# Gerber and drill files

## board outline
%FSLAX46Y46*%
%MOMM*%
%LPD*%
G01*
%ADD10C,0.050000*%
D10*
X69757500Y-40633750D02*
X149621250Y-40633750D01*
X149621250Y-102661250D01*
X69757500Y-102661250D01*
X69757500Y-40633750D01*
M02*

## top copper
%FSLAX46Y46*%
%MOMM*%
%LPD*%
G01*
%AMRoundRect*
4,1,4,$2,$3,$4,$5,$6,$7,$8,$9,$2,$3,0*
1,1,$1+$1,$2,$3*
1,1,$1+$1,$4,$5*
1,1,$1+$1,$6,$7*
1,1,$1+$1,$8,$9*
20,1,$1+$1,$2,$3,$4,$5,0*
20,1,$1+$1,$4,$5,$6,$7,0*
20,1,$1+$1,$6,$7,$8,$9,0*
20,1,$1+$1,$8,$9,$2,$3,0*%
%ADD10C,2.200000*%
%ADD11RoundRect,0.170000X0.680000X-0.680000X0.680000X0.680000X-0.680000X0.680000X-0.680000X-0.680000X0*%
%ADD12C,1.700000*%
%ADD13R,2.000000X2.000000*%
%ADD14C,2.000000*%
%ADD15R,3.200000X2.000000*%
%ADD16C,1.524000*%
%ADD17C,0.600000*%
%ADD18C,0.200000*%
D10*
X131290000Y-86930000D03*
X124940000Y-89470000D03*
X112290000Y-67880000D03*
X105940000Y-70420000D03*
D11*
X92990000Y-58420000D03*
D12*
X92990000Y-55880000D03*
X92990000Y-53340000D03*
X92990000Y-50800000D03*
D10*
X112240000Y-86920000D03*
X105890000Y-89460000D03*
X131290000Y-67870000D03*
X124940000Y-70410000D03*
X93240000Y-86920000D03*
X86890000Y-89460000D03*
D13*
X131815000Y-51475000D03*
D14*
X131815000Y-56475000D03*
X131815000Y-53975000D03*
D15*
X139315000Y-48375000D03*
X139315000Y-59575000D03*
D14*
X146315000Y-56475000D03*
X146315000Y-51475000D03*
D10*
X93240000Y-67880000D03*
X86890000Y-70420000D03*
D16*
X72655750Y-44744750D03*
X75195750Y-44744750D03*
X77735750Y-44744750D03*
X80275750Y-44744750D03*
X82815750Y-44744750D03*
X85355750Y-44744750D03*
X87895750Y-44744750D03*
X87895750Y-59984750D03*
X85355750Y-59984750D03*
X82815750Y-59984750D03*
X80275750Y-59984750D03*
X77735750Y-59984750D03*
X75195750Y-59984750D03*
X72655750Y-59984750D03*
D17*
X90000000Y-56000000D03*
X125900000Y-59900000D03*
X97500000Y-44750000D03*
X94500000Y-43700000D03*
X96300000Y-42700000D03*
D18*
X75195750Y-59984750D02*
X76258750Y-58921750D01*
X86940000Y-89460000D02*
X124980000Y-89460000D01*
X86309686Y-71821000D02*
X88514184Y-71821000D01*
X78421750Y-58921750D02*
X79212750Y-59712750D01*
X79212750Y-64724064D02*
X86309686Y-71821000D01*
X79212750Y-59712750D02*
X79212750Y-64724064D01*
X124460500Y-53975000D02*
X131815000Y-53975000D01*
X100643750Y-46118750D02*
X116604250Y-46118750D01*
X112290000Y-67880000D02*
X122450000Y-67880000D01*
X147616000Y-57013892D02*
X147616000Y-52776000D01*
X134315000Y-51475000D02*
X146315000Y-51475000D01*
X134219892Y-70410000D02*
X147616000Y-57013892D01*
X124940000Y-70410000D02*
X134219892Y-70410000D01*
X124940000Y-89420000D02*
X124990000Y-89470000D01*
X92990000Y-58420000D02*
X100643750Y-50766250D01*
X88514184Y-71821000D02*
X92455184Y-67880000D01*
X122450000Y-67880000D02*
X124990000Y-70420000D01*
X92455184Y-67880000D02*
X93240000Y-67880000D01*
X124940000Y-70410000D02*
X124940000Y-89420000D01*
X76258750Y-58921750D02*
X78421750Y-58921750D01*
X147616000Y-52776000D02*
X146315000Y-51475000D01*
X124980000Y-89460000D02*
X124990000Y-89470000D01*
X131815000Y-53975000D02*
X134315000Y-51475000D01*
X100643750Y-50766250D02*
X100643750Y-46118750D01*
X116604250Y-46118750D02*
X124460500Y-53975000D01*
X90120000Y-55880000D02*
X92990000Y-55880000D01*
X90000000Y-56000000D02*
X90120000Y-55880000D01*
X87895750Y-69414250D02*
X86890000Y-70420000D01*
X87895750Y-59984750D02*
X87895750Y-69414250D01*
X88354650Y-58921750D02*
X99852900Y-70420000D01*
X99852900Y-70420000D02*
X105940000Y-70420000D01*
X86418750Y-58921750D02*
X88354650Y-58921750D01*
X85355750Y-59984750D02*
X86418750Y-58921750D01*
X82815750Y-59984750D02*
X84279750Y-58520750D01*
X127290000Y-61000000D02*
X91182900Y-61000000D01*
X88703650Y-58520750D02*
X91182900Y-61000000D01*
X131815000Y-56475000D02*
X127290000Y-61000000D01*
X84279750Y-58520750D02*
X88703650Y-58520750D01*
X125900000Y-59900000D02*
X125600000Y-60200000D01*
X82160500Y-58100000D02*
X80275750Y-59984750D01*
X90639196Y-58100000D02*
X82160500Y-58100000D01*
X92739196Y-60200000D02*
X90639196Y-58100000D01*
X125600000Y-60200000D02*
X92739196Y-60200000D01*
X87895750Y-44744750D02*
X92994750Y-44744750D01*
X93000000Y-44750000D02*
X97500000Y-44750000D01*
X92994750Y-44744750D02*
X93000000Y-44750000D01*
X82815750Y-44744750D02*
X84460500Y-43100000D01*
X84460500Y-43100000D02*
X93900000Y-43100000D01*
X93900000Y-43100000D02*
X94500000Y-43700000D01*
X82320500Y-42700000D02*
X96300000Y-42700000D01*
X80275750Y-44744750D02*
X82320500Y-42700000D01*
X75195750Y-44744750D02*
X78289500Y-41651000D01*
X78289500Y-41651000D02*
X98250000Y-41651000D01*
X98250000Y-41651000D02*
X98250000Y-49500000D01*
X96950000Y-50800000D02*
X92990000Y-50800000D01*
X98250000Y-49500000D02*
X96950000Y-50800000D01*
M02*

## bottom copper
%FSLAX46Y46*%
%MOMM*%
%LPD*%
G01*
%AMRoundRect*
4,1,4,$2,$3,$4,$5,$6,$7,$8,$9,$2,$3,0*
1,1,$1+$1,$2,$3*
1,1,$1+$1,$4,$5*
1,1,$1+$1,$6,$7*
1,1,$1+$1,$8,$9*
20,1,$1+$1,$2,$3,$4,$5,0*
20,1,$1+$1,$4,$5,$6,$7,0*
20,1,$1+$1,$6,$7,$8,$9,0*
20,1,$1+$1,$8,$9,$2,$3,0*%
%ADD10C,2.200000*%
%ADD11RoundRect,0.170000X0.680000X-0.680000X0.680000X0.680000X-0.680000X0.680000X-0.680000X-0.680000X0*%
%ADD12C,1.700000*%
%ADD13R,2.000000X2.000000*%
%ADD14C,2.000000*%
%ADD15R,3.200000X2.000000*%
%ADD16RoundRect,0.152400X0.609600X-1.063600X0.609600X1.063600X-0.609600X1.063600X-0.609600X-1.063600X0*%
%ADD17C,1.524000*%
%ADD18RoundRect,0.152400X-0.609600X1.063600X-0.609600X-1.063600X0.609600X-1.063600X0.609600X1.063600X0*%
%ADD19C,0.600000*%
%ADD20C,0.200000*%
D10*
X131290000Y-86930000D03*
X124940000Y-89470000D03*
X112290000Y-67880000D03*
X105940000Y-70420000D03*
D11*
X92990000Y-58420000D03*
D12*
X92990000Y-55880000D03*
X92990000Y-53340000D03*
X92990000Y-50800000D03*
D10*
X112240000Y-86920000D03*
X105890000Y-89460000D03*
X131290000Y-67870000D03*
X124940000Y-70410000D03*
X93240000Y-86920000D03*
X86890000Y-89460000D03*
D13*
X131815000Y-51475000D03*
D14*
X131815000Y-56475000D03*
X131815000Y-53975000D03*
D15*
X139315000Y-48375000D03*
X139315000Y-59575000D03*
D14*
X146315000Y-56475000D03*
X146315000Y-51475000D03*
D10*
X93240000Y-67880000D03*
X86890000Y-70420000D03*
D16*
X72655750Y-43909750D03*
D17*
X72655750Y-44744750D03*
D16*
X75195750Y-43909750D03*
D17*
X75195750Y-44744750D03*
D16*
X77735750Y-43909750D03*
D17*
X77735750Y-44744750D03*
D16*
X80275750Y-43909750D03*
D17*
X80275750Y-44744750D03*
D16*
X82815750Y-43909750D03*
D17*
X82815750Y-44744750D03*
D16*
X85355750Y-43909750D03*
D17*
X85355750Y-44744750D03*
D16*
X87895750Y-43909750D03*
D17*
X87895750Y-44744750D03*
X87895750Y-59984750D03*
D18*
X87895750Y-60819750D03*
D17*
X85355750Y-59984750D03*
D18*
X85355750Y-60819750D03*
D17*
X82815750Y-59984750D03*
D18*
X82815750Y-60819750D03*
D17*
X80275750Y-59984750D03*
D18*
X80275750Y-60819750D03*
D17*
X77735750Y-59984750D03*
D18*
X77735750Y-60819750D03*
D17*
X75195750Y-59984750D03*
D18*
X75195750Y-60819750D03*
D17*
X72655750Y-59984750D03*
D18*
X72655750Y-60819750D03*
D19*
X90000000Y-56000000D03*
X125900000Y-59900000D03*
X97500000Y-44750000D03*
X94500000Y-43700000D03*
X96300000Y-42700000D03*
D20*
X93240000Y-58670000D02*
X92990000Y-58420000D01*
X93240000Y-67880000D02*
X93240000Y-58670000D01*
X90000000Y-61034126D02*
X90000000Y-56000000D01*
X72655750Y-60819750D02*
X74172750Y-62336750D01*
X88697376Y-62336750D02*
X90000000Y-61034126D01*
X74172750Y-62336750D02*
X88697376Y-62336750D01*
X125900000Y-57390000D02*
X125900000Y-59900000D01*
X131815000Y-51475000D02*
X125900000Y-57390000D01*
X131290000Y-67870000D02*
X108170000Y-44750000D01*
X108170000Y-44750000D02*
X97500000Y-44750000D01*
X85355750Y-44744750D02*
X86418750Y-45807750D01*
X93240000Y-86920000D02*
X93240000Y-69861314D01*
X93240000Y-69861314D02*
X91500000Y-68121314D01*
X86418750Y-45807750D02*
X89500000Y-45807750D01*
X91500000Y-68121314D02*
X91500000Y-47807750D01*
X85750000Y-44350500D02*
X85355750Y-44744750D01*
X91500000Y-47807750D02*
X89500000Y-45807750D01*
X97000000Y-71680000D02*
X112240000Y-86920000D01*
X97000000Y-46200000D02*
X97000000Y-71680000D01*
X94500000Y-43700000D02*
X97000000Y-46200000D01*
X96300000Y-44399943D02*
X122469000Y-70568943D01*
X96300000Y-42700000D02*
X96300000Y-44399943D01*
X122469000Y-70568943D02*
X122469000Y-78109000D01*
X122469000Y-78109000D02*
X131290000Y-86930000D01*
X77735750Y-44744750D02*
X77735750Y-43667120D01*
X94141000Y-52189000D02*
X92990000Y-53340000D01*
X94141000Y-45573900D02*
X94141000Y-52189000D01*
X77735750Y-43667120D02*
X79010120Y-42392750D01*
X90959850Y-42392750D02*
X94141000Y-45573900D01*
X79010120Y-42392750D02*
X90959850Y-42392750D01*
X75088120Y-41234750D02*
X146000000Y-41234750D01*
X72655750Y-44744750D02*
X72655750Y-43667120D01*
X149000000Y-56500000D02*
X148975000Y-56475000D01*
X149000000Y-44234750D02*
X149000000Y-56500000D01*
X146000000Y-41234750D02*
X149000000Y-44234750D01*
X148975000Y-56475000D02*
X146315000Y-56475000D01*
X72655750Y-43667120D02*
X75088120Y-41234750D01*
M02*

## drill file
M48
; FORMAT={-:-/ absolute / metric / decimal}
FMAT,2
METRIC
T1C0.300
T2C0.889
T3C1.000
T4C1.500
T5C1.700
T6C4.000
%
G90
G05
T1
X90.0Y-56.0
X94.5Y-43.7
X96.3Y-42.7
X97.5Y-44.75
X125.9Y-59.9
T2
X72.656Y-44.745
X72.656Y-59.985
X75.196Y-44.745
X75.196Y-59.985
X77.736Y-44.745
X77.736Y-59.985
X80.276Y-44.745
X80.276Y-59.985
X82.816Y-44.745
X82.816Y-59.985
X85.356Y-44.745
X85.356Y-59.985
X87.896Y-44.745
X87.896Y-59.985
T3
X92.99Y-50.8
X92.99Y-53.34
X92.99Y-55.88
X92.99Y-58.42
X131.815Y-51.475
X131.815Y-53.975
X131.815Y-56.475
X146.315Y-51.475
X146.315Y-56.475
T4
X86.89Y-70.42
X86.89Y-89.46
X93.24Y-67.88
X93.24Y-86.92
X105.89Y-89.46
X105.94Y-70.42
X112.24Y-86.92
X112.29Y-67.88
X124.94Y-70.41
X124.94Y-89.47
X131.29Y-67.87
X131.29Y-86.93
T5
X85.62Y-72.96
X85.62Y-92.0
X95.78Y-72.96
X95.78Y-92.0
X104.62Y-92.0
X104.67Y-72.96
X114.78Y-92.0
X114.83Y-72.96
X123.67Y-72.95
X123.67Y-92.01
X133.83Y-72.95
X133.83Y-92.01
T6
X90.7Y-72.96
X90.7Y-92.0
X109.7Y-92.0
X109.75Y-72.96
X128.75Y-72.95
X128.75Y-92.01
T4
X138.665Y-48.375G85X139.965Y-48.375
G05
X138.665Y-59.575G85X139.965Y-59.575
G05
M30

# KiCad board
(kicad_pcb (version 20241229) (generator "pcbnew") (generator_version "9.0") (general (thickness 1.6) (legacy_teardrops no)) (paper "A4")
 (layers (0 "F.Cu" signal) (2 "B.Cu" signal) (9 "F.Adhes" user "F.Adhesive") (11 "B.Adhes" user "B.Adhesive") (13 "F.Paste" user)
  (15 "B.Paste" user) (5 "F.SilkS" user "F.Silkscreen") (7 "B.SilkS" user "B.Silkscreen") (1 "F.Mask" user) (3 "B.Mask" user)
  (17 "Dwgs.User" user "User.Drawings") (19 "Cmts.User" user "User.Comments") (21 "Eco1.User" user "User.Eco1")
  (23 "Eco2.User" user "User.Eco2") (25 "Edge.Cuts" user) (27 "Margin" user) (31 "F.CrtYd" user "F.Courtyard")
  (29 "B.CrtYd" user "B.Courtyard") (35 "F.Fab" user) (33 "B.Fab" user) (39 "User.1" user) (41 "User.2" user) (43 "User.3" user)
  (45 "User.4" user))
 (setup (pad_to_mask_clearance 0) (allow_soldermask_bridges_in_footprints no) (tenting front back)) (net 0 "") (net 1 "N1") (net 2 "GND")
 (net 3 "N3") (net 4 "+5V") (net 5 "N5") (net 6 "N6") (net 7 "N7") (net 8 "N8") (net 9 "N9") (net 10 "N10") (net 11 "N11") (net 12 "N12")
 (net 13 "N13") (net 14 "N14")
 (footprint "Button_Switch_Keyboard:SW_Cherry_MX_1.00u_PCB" (layer "F.Cu") (at 131.29 86.93)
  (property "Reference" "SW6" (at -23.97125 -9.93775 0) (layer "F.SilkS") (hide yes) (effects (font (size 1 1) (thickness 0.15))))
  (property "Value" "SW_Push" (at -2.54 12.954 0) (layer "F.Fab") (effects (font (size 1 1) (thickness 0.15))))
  (pad "" np_thru_hole circle (at -7.62 5.08) (size 1.7 1.7) (drill 1.7) (layers "*.Cu" "*.Mask"))
  (pad "" np_thru_hole circle (at -2.54 5.08) (size 4 4) (drill 4) (layers "*.Cu" "*.Mask"))
  (pad "" np_thru_hole circle (at 2.54 5.08) (size 1.7 1.7) (drill 1.7) (layers "*.Cu" "*.Mask"))
  (pad "1" thru_hole circle (at 0 0) (size 2.2 2.2) (drill 1.5) (layers "*.Cu" "*.Mask") (remove_unused_layers no) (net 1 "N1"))
  (pad "2" thru_hole circle (at -6.35 2.54) (size 2.2 2.2) (drill 1.5) (layers "*.Cu" "*.Mask") (remove_unused_layers no) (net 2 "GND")))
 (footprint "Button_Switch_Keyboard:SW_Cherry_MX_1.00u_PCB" (layer "F.Cu") (at 112.29 67.88)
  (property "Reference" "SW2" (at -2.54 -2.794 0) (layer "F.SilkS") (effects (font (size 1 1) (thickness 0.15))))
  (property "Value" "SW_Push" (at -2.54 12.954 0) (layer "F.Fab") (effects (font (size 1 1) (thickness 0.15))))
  (pad "" np_thru_hole circle (at -7.62 5.08) (size 1.7 1.7) (drill 1.7) (layers "*.Cu" "*.Mask"))
  (pad "" np_thru_hole circle (at -2.54 5.08) (size 4 4) (drill 4) (layers "*.Cu" "*.Mask"))
  (pad "" np_thru_hole circle (at 2.54 5.08) (size 1.7 1.7) (drill 1.7) (layers "*.Cu" "*.Mask"))
  (pad "1" thru_hole circle (at 0 0) (size 2.2 2.2) (drill 1.5) (layers "*.Cu" "*.Mask") (remove_unused_layers no) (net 2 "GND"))
  (pad "2" thru_hole circle (at -6.35 2.54) (size 2.2 2.2) (drill 1.5) (layers "*.Cu" "*.Mask") (remove_unused_layers no) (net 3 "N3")))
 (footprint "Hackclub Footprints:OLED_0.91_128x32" (layer "F.Cu") (at 92.99 58.42 90)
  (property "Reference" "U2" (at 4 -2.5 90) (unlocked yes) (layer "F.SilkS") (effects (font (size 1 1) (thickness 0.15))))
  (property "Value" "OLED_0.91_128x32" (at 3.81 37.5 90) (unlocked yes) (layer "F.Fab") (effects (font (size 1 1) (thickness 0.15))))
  (pad "1" thru_hole roundrect (at 0 0 90) (size 1.7 1.7) (drill 1) (layers "*.Cu" "*.Mask") (remove_unused_layers no)
   (roundrect_rratio 0.1) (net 2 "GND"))
  (pad "2" thru_hole circle (at 2.54 0 90) (size 1.7 1.7) (drill 1) (layers "*.Cu" "*.Mask") (remove_unused_layers no) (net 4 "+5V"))
  (pad "3" thru_hole circle (at 5.08 0 90) (size 1.7 1.7) (drill 1) (layers "*.Cu" "*.Mask") (remove_unused_layers no) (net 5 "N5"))
  (pad "4" thru_hole circle (at 7.62 0 90) (size 1.7 1.7) (drill 1) (layers "*.Cu" "*.Mask") (remove_unused_layers no) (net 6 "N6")))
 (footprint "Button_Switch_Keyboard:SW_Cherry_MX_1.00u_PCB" (layer "F.Cu") (at 112.24 86.92)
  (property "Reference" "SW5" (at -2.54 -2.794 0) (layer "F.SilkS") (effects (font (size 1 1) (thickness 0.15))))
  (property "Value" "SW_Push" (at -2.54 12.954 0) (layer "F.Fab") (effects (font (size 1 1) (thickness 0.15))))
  (pad "" np_thru_hole circle (at -7.62 5.08) (size 1.7 1.7) (drill 1.7) (layers "*.Cu" "*.Mask"))
  (pad "" np_thru_hole circle (at -2.54 5.08) (size 4 4) (drill 4) (layers "*.Cu" "*.Mask"))
  (pad "" np_thru_hole circle (at 2.54 5.08) (size 1.7 1.7) (drill 1.7) (layers "*.Cu" "*.Mask"))
  (pad "1" thru_hole circle (at 0 0) (size 2.2 2.2) (drill 1.5) (layers "*.Cu" "*.Mask") (remove_unused_layers no) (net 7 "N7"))
  (pad "2" thru_hole circle (at -6.35 2.54) (size 2.2 2.2) (drill 1.5) (layers "*.Cu" "*.Mask") (remove_unused_layers no) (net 2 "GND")))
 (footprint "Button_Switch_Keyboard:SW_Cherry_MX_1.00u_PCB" (layer "F.Cu") (at 131.29 67.87)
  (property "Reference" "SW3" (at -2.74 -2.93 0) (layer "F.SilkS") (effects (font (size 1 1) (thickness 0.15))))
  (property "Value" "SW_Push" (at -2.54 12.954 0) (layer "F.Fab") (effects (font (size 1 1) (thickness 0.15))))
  (pad "" np_thru_hole circle (at -7.62 5.08) (size 1.7 1.7) (drill 1.7) (layers "*.Cu" "*.Mask"))
  (pad "" np_thru_hole circle (at -2.54 5.08) (size 4 4) (drill 4) (layers "*.Cu" "*.Mask"))
  (pad "" np_thru_hole circle (at 2.54 5.08) (size 1.7 1.7) (drill 1.7) (layers "*.Cu" "*.Mask"))
  (pad "1" thru_hole circle (at 0 0) (size 2.2 2.2) (drill 1.5) (layers "*.Cu" "*.Mask") (remove_unused_layers no) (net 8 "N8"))
  (pad "2" thru_hole circle (at -6.35 2.54) (size 2.2 2.2) (drill 1.5) (layers "*.Cu" "*.Mask") (remove_unused_layers no) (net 2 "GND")))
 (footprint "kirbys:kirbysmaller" (layer "F.Cu") (at 80 51.5)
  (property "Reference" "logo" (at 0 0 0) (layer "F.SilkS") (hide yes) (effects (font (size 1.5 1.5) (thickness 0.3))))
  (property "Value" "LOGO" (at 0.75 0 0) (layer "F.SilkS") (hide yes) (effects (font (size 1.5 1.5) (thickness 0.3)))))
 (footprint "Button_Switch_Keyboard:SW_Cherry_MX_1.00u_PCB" (layer "F.Cu") (at 93.24 86.92)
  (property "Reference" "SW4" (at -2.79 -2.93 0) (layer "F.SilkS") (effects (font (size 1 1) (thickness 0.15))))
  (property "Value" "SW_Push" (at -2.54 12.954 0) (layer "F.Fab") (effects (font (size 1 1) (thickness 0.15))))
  (pad "" np_thru_hole circle (at -7.62 5.08) (size 1.7 1.7) (drill 1.7) (layers "*.Cu" "*.Mask"))
  (pad "" np_thru_hole circle (at -2.54 5.08) (size 4 4) (drill 4) (layers "*.Cu" "*.Mask"))
  (pad "" np_thru_hole circle (at 2.54 5.08) (size 1.7 1.7) (drill 1.7) (layers "*.Cu" "*.Mask"))
  (pad "1" thru_hole circle (at 0 0) (size 2.2 2.2) (drill 1.5) (layers "*.Cu" "*.Mask") (remove_unused_layers no) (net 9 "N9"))
  (pad "2" thru_hole circle (at -6.35 2.54) (size 2.2 2.2) (drill 1.5) (layers "*.Cu" "*.Mask") (remove_unused_layers no) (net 2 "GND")))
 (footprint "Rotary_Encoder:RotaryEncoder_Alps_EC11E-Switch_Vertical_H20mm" (layer "F.Cu") (at 131.815 51.475)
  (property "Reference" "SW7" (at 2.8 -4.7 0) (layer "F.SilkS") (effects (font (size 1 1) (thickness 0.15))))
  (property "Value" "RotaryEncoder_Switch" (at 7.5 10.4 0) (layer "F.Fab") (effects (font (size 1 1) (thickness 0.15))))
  (pad "A" thru_hole rect (at 0 0) (size 2 2) (drill 1) (layers "*.Cu" "*.Mask") (remove_unused_layers no) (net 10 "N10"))
  (pad "B" thru_hole circle (at 0 5) (size 2 2) (drill 1) (layers "*.Cu" "*.Mask") (remove_unused_layers no) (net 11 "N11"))
  (pad "C" thru_hole circle (at 0 2.5) (size 2 2) (drill 1) (layers "*.Cu" "*.Mask") (remove_unused_layers no) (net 2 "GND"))
  (pad "MP" thru_hole rect (at 7.5 -3.1) (size 3.2 2) (drill oval 2.8 1.5) (layers "*.Cu" "*.Mask") (remove_unused_layers no))
  (pad "MP" thru_hole rect (at 7.5 8.1) (size 3.2 2) (drill oval 2.8 1.5) (layers "*.Cu" "*.Mask") (remove_unused_layers no))
  (pad "S1" thru_hole circle (at 14.5 5) (size 2 2) (drill 1) (layers "*.Cu" "*.Mask") (remove_unused_layers no) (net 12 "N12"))
  (pad "S2" thru_hole circle (at 14.5 0) (size 2 2) (drill 1) (layers "*.Cu" "*.Mask") (remove_unused_layers no) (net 2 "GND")))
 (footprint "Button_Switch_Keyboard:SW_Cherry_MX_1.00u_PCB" (layer "F.Cu") (at 93.24 67.88)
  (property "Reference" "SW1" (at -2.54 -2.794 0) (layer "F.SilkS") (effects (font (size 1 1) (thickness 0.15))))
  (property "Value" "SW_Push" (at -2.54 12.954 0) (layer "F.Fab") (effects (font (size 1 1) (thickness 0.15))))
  (pad "" np_thru_hole circle (at -7.62 5.08) (size 1.7 1.7) (drill 1.7) (layers "*.Cu" "*.Mask"))
  (pad "" np_thru_hole circle (at -2.54 5.08) (size 4 4) (drill 4) (layers "*.Cu" "*.Mask"))
  (pad "" np_thru_hole circle (at 2.54 5.08) (size 1.7 1.7) (drill 1.7) (layers "*.Cu" "*.Mask"))
  (pad "1" thru_hole circle (at 0 0) (size 2.2 2.2) (drill 1.5) (layers "*.Cu" "*.Mask") (remove_unused_layers no) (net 2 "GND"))
  (pad "2" thru_hole circle (at -6.35 2.54) (size 2.2 2.2) (drill 1.5) (layers "*.Cu" "*.Mask") (remove_unused_layers no) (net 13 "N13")))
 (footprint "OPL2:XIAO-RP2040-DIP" (layer "B.Cu") (at 80.27575 52.36475 -90)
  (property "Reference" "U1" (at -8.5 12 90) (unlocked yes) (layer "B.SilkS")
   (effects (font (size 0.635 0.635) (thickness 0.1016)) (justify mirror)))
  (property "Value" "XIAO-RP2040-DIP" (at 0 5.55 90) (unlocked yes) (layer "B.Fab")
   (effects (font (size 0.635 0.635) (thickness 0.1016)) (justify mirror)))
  (pad "1" smd roundrect (at -8.455 7.62 90) (size 2.432 1.524) (layers "B.Cu" "B.Mask") (roundrect_rratio 0.1) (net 12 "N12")
   (thermal_bridge_angle 45))
  (pad "1" thru_hole circle (at -7.62 7.62 90) (size 1.524 1.524) (drill 0.889) (layers "*.Cu" "*.Mask") (remove_unused_layers no)
   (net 12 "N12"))
  (pad "2" smd roundrect (at -8.455 5.08 90) (size 2.432 1.524) (layers "B.Cu" "B.Mask") (roundrect_rratio 0.1) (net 6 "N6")
   (thermal_bridge_angle 45))
  (pad "2" thru_hole circle (at -7.62 5.08 90) (size 1.524 1.524) (drill 0.889) (layers "*.Cu" "*.Mask") (remove_unused_layers no)
   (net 6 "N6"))
  (pad "3" smd roundrect (at -8.455 2.54 90) (size 2.432 1.524) (layers "B.Cu" "B.Mask") (roundrect_rratio 0.1) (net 5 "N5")
   (thermal_bridge_angle 45))
  (pad "3" thru_hole circle (at -7.62 2.54 90) (size 1.524 1.524) (drill 0.889) (layers "*.Cu" "*.Mask") (remove_unused_layers no)
   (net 5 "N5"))
  (pad "4" smd roundrect (at -8.455 0 90) (size 2.432 1.524) (layers "B.Cu" "B.Mask") (roundrect_rratio 0.1) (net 1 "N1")
   (thermal_bridge_angle 45))
  (pad "4" thru_hole circle (at -7.62 0 90) (size 1.524 1.524) (drill 0.889) (layers "*.Cu" "*.Mask") (remove_unused_layers no) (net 1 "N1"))
  (pad "5" smd roundrect (at -8.455 -2.54 90) (size 2.432 1.524) (layers "B.Cu" "B.Mask") (roundrect_rratio 0.1) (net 7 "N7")
   (thermal_bridge_angle 45))
  (pad "5" thru_hole circle (at -7.62 -2.54 90) (size 1.524 1.524) (drill 0.889) (layers "*.Cu" "*.Mask") (remove_unused_layers no)
   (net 7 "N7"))
  (pad "6" smd roundrect (at -8.455 -5.08 90) (size 2.432 1.524) (layers "B.Cu" "B.Mask") (roundrect_rratio 0.1) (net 9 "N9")
   (thermal_bridge_angle 45))
  (pad "6" thru_hole circle (at -7.62 -5.08 90) (size 1.524 1.524) (drill 0.889) (layers "*.Cu" "*.Mask") (remove_unused_layers no)
   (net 9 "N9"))
  (pad "7" smd roundrect (at -8.455 -7.62 90) (size 2.432 1.524) (layers "B.Cu" "B.Mask") (roundrect_rratio 0.1) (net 8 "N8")
   (thermal_bridge_angle 45))
  (pad "7" thru_hole circle (at -7.62 -7.62 90) (size 1.524 1.524) (drill 0.889) (layers "*.Cu" "*.Mask") (remove_unused_layers no)
   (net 8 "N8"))
  (pad "8" thru_hole circle (at 7.62 -7.62 270) (size 1.524 1.524) (drill 0.889) (layers "*.Cu" "*.Mask") (remove_unused_layers no)
   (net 13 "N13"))
  (pad "8" smd roundrect (at 8.455 -7.62 270) (size 2.432 1.524) (layers "B.Cu" "B.Mask") (roundrect_rratio 0.1) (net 13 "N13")
   (thermal_bridge_angle 45))
  (pad "9" thru_hole circle (at 7.62 -5.08 270) (size 1.524 1.524) (drill 0.889) (layers "*.Cu" "*.Mask") (remove_unused_layers no)
   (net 3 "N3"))
  (pad "9" smd roundrect (at 8.455 -5.08 270) (size 2.432 1.524) (layers "B.Cu" "B.Mask") (roundrect_rratio 0.1) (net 3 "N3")
   (thermal_bridge_angle 45))
  (pad "10" thru_hole circle (at 7.62 -2.54 270) (size 1.524 1.524) (drill 0.889) (layers "*.Cu" "*.Mask") (remove_unused_layers no)
   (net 11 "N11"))
  (pad "10" smd roundrect (at 8.455 -2.54 270) (size 2.432 1.524) (layers "B.Cu" "B.Mask") (roundrect_rratio 0.1) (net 11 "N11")
   (thermal_bridge_angle 45))
  (pad "11" thru_hole circle (at 7.62 0 270) (size 1.524 1.524) (drill 0.889) (layers "*.Cu" "*.Mask") (remove_unused_layers no)
   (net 10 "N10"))
  (pad "11" smd roundrect (at 8.455 0 270) (size 2.432 1.524) (layers "B.Cu" "B.Mask") (roundrect_rratio 0.1) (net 10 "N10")
   (thermal_bridge_angle 45))
  (pad "12" thru_hole circle (at 7.62 2.54 270) (size 1.524 1.524) (drill 0.889) (layers "*.Cu" "*.Mask") (remove_unused_layers no)
   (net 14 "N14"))
  (pad "12" smd roundrect (at 8.455 2.54 270) (size 2.432 1.524) (layers "B.Cu" "B.Mask") (roundrect_rratio 0.1) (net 14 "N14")
   (thermal_bridge_angle 45))
  (pad "13" thru_hole circle (at 7.62 5.08 270) (size 1.524 1.524) (drill 0.889) (layers "*.Cu" "*.Mask") (remove_unused_layers no)
   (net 2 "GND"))
  (pad "13" smd roundrect (at 8.455 5.08 270) (size 2.432 1.524) (layers "B.Cu" "B.Mask") (roundrect_rratio 0.1) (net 2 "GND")
   (thermal_bridge_angle 45))
  (pad "14" thru_hole circle (at 7.62 7.62 270) (size 1.524 1.524) (drill 0.889) (layers "*.Cu" "*.Mask") (remove_unused_layers no)
   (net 4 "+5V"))
  (pad "14" smd roundrect (at 8.455 7.62 270) (size 2.432 1.524) (layers "B.Cu" "B.Mask") (roundrect_rratio 0.1) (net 4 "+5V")
   (thermal_bridge_angle 45)))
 (gr_rect (start 69.7575 40.63375) (end 149.62125 102.66125) (stroke (width 0.05) (type default)) (fill no) (layer "Edge.Cuts"))
 (segment (start 75.19575 59.98475) (end 76.25875 58.92175) (width 0.2) (layer "F.Cu") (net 2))
 (segment (start 86.94 89.46) (end 124.98 89.46) (width 0.2) (layer "F.Cu") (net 2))
 (segment (start 86.309686 71.821) (end 88.514184 71.821) (width 0.2) (layer "F.Cu") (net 2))
 (segment (start 78.42175 58.92175) (end 79.21275 59.71275) (width 0.2) (layer "F.Cu") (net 2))
 (segment (start 79.21275 64.724064) (end 86.309686 71.821) (width 0.2) (layer "F.Cu") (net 2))
 (segment (start 79.21275 59.71275) (end 79.21275 64.724064) (width 0.2) (layer "F.Cu") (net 2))
 (segment (start 124.4605 53.975) (end 131.815 53.975) (width 0.2) (layer "F.Cu") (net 2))
 (segment (start 100.64375 46.11875) (end 116.60425 46.11875) (width 0.2) (layer "F.Cu") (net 2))
 (segment (start 112.29 67.88) (end 122.45 67.88) (width 0.2) (layer "F.Cu") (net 2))
 (segment (start 147.616 57.013892) (end 147.616 52.776) (width 0.2) (layer "F.Cu") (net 2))
 (segment (start 134.315 51.475) (end 146.315 51.475) (width 0.2) (layer "F.Cu") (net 2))
 (segment (start 134.219892 70.41) (end 147.616 57.013892) (width 0.2) (layer "F.Cu") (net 2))
 (segment (start 124.94 70.41) (end 134.219892 70.41) (width 0.2) (layer "F.Cu") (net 2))
 (segment (start 124.94 89.42) (end 124.99 89.47) (width 0.2) (layer "F.Cu") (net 2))
 (segment (start 92.99 58.42) (end 100.64375 50.76625) (width 0.2) (layer "F.Cu") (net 2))
 (segment (start 88.514184 71.821) (end 92.455184 67.88) (width 0.2) (layer "F.Cu") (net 2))
 (segment (start 122.45 67.88) (end 124.99 70.42) (width 0.2) (layer "F.Cu") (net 2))
 (segment (start 92.455184 67.88) (end 93.24 67.88) (width 0.2) (layer "F.Cu") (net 2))
 (segment (start 124.94 70.41) (end 124.94 89.42) (width 0.2) (layer "F.Cu") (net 2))
 (segment (start 76.25875 58.92175) (end 78.42175 58.92175) (width 0.2) (layer "F.Cu") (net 2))
 (segment (start 147.616 52.776) (end 146.315 51.475) (width 0.2) (layer "F.Cu") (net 2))
 (segment (start 124.98 89.46) (end 124.99 89.47) (width 0.2) (layer "F.Cu") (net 2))
 (segment (start 131.815 53.975) (end 134.315 51.475) (width 0.2) (layer "F.Cu") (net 2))
 (segment (start 100.64375 50.76625) (end 100.64375 46.11875) (width 0.2) (layer "F.Cu") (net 2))
 (segment (start 116.60425 46.11875) (end 124.4605 53.975) (width 0.2) (layer "F.Cu") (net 2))
 (segment (start 93.24 58.67) (end 92.99 58.42) (width 0.2) (layer "B.Cu") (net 2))
 (segment (start 93.24 67.88) (end 93.24 58.67) (width 0.2) (layer "B.Cu") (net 2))
 (segment (start 90.12 55.88) (end 92.99 55.88) (width 0.2) (layer "F.Cu") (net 4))
 (segment (start 90 56) (end 90.12 55.88) (width 0.2) (layer "F.Cu") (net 4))
 (via (at 90 56) (size 0.6) (drill 0.3) (layers "F.Cu" "B.Cu") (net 4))
 (segment (start 90 61.034126) (end 90 56) (width 0.2) (layer "B.Cu") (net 4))
 (segment (start 72.65575 60.81975) (end 74.17275 62.33675) (width 0.2) (layer "B.Cu") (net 4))
 (segment (start 88.697376 62.33675) (end 90 61.034126) (width 0.2) (layer "B.Cu") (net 4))
 (segment (start 74.17275 62.33675) (end 88.697376 62.33675) (width 0.2) (layer "B.Cu") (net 4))
 (segment (start 87.89575 69.41425) (end 86.89 70.42) (width 0.2) (layer "F.Cu") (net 13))
 (segment (start 87.89575 59.98475) (end 87.89575 69.41425) (width 0.2) (layer "F.Cu") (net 13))
 (segment (start 88.35465 58.92175) (end 99.8529 70.42) (width 0.2) (layer "F.Cu") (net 3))
 (segment (start 99.8529 70.42) (end 105.94 70.42) (width 0.2) (layer "F.Cu") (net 3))
 (segment (start 86.41875 58.92175) (end 88.35465 58.92175) (width 0.2) (layer "F.Cu") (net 3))
 (segment (start 85.35575 59.98475) (end 86.41875 58.92175) (width 0.2) (layer "F.Cu") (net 3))
 (segment (start 82.81575 59.98475) (end 84.27975 58.52075) (width 0.2) (layer "F.Cu") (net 11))
 (segment (start 127.29 61) (end 91.1829 61) (width 0.2) (layer "F.Cu") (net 11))
 (segment (start 88.70365 58.52075) (end 91.1829 61) (width 0.2) (layer "F.Cu") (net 11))
 (segment (start 131.815 56.475) (end 127.29 61) (width 0.2) (layer "F.Cu") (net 11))
 (segment (start 84.27975 58.52075) (end 88.70365 58.52075) (width 0.2) (layer "F.Cu") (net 11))
 (segment (start 125.9 59.9) (end 125.6 60.2) (width 0.2) (layer "F.Cu") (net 10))
 (segment (start 82.1605 58.1) (end 80.27575 59.98475) (width 0.2) (layer "F.Cu") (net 10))
 (segment (start 90.639196 58.1) (end 82.1605 58.1) (width 0.2) (layer "F.Cu") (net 10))
 (segment (start 92.739196 60.2) (end 90.639196 58.1) (width 0.2) (layer "F.Cu") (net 10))
 (segment (start 125.6 60.2) (end 92.739196 60.2) (width 0.2) (layer "F.Cu") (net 10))
 (via (at 125.9 59.9) (size 0.6) (drill 0.3) (layers "F.Cu" "B.Cu") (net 10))
 (segment (start 125.9 57.39) (end 125.9 59.9) (width 0.2) (layer "B.Cu") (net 10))
 (segment (start 131.815 51.475) (end 125.9 57.39) (width 0.2) (layer "B.Cu") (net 10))
 (segment (start 87.89575 44.74475) (end 92.99475 44.74475) (width 0.2) (layer "F.Cu") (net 8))
 (segment (start 93 44.75) (end 97.5 44.75) (width 0.2) (layer "F.Cu") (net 8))
 (segment (start 92.99475 44.74475) (end 93 44.75) (width 0.2) (layer "F.Cu") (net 8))
 (via (at 97.5 44.75) (size 0.6) (drill 0.3) (layers "F.Cu" "B.Cu") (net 8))
 (segment (start 131.29 67.87) (end 108.17 44.75) (width 0.2) (layer "B.Cu") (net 8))
 (segment (start 108.17 44.75) (end 97.5 44.75) (width 0.2) (layer "B.Cu") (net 8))
 (segment (start 85.35575 44.74475) (end 86.41875 45.80775) (width 0.2) (layer "B.Cu") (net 9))
 (segment (start 93.24 86.92) (end 93.24 69.861314) (width 0.2) (layer "B.Cu") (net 9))
 (segment (start 93.24 69.861314) (end 91.5 68.121314) (width 0.2) (layer "B.Cu") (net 9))
 (segment (start 86.41875 45.80775) (end 89.5 45.80775) (width 0.2) (layer "B.Cu") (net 9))
 (segment (start 91.5 68.121314) (end 91.5 47.80775) (width 0.2) (layer "B.Cu") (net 9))
 (segment (start 85.75 44.3505) (end 85.35575 44.74475) (width 0.2) (layer "B.Cu") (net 9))
 (segment (start 91.5 47.80775) (end 89.5 45.80775) (width 0.2) (layer "B.Cu") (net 9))
 (segment (start 82.81575 44.74475) (end 84.4605 43.1) (width 0.2) (layer "F.Cu") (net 7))
 (segment (start 84.4605 43.1) (end 93.9 43.1) (width 0.2) (layer "F.Cu") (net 7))
 (segment (start 93.9 43.1) (end 94.5 43.7) (width 0.2) (layer "F.Cu") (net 7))
 (via (at 94.5 43.7) (size 0.6) (drill 0.3) (layers "F.Cu" "B.Cu") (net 7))
 (segment (start 97 71.68) (end 112.24 86.92) (width 0.2) (layer "B.Cu") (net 7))
 (segment (start 97 46.2) (end 97 71.68) (width 0.2) (layer "B.Cu") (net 7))
 (segment (start 94.5 43.7) (end 97 46.2) (width 0.2) (layer "B.Cu") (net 7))
 (segment (start 82.3205 42.7) (end 96.3 42.7) (width 0.2) (layer "F.Cu") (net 1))
 (segment (start 80.27575 44.74475) (end 82.3205 42.7) (width 0.2) (layer "F.Cu") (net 1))
 (via (at 96.3 42.7) (size 0.6) (drill 0.3) (layers "F.Cu" "B.Cu") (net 1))
 (segment (start 96.3 44.399943) (end 122.469 70.568943) (width 0.2) (layer "B.Cu") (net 1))
 (segment (start 96.3 42.7) (end 96.3 44.399943) (width 0.2) (layer "B.Cu") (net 1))
 (segment (start 122.469 70.568943) (end 122.469 78.109) (width 0.2) (layer "B.Cu") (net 1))
 (segment (start 122.469 78.109) (end 131.29 86.93) (width 0.2) (layer "B.Cu") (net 1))
 (segment (start 77.73575 44.74475) (end 77.73575 43.66712) (width 0.2) (layer "B.Cu") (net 5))
 (segment (start 94.141 52.189) (end 92.99 53.34) (width 0.2) (layer "B.Cu") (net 5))
 (segment (start 94.141 45.5739) (end 94.141 52.189) (width 0.2) (layer "B.Cu") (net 5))
 (segment (start 77.73575 43.66712) (end 79.01012 42.39275) (width 0.2) (layer "B.Cu") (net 5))
 (segment (start 90.95985 42.39275) (end 94.141 45.5739) (width 0.2) (layer "B.Cu") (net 5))
 (segment (start 79.01012 42.39275) (end 90.95985 42.39275) (width 0.2) (layer "B.Cu") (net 5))
 (segment (start 75.19575 44.74475) (end 78.2895 41.651) (width 0.2) (layer "F.Cu") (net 6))
 (segment (start 78.2895 41.651) (end 98.25 41.651) (width 0.2) (layer "F.Cu") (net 6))
 (segment (start 98.25 41.651) (end 98.25 49.5) (width 0.2) (layer "F.Cu") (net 6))
 (segment (start 96.95 50.8) (end 92.99 50.8) (width 0.2) (layer "F.Cu") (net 6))
 (segment (start 98.25 49.5) (end 96.95 50.8) (width 0.2) (layer "F.Cu") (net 6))
 (segment (start 75.08812 41.23475) (end 146 41.23475) (width 0.2) (layer "B.Cu") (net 12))
 (segment (start 72.65575 44.74475) (end 72.65575 43.66712) (width 0.2) (layer "B.Cu") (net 12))
 (segment (start 149 56.5) (end 148.975 56.475) (width 0.2) (layer "B.Cu") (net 12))
 (segment (start 149 44.23475) (end 149 56.5) (width 0.2) (layer "B.Cu") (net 12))
 (segment (start 146 41.23475) (end 149 44.23475) (width 0.2) (layer "B.Cu") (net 12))
 (segment (start 148.975 56.475) (end 146.315 56.475) (width 0.2) (layer "B.Cu") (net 12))
 (segment (start 72.65575 43.66712) (end 75.08812 41.23475) (width 0.2) (layer "B.Cu") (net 12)))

